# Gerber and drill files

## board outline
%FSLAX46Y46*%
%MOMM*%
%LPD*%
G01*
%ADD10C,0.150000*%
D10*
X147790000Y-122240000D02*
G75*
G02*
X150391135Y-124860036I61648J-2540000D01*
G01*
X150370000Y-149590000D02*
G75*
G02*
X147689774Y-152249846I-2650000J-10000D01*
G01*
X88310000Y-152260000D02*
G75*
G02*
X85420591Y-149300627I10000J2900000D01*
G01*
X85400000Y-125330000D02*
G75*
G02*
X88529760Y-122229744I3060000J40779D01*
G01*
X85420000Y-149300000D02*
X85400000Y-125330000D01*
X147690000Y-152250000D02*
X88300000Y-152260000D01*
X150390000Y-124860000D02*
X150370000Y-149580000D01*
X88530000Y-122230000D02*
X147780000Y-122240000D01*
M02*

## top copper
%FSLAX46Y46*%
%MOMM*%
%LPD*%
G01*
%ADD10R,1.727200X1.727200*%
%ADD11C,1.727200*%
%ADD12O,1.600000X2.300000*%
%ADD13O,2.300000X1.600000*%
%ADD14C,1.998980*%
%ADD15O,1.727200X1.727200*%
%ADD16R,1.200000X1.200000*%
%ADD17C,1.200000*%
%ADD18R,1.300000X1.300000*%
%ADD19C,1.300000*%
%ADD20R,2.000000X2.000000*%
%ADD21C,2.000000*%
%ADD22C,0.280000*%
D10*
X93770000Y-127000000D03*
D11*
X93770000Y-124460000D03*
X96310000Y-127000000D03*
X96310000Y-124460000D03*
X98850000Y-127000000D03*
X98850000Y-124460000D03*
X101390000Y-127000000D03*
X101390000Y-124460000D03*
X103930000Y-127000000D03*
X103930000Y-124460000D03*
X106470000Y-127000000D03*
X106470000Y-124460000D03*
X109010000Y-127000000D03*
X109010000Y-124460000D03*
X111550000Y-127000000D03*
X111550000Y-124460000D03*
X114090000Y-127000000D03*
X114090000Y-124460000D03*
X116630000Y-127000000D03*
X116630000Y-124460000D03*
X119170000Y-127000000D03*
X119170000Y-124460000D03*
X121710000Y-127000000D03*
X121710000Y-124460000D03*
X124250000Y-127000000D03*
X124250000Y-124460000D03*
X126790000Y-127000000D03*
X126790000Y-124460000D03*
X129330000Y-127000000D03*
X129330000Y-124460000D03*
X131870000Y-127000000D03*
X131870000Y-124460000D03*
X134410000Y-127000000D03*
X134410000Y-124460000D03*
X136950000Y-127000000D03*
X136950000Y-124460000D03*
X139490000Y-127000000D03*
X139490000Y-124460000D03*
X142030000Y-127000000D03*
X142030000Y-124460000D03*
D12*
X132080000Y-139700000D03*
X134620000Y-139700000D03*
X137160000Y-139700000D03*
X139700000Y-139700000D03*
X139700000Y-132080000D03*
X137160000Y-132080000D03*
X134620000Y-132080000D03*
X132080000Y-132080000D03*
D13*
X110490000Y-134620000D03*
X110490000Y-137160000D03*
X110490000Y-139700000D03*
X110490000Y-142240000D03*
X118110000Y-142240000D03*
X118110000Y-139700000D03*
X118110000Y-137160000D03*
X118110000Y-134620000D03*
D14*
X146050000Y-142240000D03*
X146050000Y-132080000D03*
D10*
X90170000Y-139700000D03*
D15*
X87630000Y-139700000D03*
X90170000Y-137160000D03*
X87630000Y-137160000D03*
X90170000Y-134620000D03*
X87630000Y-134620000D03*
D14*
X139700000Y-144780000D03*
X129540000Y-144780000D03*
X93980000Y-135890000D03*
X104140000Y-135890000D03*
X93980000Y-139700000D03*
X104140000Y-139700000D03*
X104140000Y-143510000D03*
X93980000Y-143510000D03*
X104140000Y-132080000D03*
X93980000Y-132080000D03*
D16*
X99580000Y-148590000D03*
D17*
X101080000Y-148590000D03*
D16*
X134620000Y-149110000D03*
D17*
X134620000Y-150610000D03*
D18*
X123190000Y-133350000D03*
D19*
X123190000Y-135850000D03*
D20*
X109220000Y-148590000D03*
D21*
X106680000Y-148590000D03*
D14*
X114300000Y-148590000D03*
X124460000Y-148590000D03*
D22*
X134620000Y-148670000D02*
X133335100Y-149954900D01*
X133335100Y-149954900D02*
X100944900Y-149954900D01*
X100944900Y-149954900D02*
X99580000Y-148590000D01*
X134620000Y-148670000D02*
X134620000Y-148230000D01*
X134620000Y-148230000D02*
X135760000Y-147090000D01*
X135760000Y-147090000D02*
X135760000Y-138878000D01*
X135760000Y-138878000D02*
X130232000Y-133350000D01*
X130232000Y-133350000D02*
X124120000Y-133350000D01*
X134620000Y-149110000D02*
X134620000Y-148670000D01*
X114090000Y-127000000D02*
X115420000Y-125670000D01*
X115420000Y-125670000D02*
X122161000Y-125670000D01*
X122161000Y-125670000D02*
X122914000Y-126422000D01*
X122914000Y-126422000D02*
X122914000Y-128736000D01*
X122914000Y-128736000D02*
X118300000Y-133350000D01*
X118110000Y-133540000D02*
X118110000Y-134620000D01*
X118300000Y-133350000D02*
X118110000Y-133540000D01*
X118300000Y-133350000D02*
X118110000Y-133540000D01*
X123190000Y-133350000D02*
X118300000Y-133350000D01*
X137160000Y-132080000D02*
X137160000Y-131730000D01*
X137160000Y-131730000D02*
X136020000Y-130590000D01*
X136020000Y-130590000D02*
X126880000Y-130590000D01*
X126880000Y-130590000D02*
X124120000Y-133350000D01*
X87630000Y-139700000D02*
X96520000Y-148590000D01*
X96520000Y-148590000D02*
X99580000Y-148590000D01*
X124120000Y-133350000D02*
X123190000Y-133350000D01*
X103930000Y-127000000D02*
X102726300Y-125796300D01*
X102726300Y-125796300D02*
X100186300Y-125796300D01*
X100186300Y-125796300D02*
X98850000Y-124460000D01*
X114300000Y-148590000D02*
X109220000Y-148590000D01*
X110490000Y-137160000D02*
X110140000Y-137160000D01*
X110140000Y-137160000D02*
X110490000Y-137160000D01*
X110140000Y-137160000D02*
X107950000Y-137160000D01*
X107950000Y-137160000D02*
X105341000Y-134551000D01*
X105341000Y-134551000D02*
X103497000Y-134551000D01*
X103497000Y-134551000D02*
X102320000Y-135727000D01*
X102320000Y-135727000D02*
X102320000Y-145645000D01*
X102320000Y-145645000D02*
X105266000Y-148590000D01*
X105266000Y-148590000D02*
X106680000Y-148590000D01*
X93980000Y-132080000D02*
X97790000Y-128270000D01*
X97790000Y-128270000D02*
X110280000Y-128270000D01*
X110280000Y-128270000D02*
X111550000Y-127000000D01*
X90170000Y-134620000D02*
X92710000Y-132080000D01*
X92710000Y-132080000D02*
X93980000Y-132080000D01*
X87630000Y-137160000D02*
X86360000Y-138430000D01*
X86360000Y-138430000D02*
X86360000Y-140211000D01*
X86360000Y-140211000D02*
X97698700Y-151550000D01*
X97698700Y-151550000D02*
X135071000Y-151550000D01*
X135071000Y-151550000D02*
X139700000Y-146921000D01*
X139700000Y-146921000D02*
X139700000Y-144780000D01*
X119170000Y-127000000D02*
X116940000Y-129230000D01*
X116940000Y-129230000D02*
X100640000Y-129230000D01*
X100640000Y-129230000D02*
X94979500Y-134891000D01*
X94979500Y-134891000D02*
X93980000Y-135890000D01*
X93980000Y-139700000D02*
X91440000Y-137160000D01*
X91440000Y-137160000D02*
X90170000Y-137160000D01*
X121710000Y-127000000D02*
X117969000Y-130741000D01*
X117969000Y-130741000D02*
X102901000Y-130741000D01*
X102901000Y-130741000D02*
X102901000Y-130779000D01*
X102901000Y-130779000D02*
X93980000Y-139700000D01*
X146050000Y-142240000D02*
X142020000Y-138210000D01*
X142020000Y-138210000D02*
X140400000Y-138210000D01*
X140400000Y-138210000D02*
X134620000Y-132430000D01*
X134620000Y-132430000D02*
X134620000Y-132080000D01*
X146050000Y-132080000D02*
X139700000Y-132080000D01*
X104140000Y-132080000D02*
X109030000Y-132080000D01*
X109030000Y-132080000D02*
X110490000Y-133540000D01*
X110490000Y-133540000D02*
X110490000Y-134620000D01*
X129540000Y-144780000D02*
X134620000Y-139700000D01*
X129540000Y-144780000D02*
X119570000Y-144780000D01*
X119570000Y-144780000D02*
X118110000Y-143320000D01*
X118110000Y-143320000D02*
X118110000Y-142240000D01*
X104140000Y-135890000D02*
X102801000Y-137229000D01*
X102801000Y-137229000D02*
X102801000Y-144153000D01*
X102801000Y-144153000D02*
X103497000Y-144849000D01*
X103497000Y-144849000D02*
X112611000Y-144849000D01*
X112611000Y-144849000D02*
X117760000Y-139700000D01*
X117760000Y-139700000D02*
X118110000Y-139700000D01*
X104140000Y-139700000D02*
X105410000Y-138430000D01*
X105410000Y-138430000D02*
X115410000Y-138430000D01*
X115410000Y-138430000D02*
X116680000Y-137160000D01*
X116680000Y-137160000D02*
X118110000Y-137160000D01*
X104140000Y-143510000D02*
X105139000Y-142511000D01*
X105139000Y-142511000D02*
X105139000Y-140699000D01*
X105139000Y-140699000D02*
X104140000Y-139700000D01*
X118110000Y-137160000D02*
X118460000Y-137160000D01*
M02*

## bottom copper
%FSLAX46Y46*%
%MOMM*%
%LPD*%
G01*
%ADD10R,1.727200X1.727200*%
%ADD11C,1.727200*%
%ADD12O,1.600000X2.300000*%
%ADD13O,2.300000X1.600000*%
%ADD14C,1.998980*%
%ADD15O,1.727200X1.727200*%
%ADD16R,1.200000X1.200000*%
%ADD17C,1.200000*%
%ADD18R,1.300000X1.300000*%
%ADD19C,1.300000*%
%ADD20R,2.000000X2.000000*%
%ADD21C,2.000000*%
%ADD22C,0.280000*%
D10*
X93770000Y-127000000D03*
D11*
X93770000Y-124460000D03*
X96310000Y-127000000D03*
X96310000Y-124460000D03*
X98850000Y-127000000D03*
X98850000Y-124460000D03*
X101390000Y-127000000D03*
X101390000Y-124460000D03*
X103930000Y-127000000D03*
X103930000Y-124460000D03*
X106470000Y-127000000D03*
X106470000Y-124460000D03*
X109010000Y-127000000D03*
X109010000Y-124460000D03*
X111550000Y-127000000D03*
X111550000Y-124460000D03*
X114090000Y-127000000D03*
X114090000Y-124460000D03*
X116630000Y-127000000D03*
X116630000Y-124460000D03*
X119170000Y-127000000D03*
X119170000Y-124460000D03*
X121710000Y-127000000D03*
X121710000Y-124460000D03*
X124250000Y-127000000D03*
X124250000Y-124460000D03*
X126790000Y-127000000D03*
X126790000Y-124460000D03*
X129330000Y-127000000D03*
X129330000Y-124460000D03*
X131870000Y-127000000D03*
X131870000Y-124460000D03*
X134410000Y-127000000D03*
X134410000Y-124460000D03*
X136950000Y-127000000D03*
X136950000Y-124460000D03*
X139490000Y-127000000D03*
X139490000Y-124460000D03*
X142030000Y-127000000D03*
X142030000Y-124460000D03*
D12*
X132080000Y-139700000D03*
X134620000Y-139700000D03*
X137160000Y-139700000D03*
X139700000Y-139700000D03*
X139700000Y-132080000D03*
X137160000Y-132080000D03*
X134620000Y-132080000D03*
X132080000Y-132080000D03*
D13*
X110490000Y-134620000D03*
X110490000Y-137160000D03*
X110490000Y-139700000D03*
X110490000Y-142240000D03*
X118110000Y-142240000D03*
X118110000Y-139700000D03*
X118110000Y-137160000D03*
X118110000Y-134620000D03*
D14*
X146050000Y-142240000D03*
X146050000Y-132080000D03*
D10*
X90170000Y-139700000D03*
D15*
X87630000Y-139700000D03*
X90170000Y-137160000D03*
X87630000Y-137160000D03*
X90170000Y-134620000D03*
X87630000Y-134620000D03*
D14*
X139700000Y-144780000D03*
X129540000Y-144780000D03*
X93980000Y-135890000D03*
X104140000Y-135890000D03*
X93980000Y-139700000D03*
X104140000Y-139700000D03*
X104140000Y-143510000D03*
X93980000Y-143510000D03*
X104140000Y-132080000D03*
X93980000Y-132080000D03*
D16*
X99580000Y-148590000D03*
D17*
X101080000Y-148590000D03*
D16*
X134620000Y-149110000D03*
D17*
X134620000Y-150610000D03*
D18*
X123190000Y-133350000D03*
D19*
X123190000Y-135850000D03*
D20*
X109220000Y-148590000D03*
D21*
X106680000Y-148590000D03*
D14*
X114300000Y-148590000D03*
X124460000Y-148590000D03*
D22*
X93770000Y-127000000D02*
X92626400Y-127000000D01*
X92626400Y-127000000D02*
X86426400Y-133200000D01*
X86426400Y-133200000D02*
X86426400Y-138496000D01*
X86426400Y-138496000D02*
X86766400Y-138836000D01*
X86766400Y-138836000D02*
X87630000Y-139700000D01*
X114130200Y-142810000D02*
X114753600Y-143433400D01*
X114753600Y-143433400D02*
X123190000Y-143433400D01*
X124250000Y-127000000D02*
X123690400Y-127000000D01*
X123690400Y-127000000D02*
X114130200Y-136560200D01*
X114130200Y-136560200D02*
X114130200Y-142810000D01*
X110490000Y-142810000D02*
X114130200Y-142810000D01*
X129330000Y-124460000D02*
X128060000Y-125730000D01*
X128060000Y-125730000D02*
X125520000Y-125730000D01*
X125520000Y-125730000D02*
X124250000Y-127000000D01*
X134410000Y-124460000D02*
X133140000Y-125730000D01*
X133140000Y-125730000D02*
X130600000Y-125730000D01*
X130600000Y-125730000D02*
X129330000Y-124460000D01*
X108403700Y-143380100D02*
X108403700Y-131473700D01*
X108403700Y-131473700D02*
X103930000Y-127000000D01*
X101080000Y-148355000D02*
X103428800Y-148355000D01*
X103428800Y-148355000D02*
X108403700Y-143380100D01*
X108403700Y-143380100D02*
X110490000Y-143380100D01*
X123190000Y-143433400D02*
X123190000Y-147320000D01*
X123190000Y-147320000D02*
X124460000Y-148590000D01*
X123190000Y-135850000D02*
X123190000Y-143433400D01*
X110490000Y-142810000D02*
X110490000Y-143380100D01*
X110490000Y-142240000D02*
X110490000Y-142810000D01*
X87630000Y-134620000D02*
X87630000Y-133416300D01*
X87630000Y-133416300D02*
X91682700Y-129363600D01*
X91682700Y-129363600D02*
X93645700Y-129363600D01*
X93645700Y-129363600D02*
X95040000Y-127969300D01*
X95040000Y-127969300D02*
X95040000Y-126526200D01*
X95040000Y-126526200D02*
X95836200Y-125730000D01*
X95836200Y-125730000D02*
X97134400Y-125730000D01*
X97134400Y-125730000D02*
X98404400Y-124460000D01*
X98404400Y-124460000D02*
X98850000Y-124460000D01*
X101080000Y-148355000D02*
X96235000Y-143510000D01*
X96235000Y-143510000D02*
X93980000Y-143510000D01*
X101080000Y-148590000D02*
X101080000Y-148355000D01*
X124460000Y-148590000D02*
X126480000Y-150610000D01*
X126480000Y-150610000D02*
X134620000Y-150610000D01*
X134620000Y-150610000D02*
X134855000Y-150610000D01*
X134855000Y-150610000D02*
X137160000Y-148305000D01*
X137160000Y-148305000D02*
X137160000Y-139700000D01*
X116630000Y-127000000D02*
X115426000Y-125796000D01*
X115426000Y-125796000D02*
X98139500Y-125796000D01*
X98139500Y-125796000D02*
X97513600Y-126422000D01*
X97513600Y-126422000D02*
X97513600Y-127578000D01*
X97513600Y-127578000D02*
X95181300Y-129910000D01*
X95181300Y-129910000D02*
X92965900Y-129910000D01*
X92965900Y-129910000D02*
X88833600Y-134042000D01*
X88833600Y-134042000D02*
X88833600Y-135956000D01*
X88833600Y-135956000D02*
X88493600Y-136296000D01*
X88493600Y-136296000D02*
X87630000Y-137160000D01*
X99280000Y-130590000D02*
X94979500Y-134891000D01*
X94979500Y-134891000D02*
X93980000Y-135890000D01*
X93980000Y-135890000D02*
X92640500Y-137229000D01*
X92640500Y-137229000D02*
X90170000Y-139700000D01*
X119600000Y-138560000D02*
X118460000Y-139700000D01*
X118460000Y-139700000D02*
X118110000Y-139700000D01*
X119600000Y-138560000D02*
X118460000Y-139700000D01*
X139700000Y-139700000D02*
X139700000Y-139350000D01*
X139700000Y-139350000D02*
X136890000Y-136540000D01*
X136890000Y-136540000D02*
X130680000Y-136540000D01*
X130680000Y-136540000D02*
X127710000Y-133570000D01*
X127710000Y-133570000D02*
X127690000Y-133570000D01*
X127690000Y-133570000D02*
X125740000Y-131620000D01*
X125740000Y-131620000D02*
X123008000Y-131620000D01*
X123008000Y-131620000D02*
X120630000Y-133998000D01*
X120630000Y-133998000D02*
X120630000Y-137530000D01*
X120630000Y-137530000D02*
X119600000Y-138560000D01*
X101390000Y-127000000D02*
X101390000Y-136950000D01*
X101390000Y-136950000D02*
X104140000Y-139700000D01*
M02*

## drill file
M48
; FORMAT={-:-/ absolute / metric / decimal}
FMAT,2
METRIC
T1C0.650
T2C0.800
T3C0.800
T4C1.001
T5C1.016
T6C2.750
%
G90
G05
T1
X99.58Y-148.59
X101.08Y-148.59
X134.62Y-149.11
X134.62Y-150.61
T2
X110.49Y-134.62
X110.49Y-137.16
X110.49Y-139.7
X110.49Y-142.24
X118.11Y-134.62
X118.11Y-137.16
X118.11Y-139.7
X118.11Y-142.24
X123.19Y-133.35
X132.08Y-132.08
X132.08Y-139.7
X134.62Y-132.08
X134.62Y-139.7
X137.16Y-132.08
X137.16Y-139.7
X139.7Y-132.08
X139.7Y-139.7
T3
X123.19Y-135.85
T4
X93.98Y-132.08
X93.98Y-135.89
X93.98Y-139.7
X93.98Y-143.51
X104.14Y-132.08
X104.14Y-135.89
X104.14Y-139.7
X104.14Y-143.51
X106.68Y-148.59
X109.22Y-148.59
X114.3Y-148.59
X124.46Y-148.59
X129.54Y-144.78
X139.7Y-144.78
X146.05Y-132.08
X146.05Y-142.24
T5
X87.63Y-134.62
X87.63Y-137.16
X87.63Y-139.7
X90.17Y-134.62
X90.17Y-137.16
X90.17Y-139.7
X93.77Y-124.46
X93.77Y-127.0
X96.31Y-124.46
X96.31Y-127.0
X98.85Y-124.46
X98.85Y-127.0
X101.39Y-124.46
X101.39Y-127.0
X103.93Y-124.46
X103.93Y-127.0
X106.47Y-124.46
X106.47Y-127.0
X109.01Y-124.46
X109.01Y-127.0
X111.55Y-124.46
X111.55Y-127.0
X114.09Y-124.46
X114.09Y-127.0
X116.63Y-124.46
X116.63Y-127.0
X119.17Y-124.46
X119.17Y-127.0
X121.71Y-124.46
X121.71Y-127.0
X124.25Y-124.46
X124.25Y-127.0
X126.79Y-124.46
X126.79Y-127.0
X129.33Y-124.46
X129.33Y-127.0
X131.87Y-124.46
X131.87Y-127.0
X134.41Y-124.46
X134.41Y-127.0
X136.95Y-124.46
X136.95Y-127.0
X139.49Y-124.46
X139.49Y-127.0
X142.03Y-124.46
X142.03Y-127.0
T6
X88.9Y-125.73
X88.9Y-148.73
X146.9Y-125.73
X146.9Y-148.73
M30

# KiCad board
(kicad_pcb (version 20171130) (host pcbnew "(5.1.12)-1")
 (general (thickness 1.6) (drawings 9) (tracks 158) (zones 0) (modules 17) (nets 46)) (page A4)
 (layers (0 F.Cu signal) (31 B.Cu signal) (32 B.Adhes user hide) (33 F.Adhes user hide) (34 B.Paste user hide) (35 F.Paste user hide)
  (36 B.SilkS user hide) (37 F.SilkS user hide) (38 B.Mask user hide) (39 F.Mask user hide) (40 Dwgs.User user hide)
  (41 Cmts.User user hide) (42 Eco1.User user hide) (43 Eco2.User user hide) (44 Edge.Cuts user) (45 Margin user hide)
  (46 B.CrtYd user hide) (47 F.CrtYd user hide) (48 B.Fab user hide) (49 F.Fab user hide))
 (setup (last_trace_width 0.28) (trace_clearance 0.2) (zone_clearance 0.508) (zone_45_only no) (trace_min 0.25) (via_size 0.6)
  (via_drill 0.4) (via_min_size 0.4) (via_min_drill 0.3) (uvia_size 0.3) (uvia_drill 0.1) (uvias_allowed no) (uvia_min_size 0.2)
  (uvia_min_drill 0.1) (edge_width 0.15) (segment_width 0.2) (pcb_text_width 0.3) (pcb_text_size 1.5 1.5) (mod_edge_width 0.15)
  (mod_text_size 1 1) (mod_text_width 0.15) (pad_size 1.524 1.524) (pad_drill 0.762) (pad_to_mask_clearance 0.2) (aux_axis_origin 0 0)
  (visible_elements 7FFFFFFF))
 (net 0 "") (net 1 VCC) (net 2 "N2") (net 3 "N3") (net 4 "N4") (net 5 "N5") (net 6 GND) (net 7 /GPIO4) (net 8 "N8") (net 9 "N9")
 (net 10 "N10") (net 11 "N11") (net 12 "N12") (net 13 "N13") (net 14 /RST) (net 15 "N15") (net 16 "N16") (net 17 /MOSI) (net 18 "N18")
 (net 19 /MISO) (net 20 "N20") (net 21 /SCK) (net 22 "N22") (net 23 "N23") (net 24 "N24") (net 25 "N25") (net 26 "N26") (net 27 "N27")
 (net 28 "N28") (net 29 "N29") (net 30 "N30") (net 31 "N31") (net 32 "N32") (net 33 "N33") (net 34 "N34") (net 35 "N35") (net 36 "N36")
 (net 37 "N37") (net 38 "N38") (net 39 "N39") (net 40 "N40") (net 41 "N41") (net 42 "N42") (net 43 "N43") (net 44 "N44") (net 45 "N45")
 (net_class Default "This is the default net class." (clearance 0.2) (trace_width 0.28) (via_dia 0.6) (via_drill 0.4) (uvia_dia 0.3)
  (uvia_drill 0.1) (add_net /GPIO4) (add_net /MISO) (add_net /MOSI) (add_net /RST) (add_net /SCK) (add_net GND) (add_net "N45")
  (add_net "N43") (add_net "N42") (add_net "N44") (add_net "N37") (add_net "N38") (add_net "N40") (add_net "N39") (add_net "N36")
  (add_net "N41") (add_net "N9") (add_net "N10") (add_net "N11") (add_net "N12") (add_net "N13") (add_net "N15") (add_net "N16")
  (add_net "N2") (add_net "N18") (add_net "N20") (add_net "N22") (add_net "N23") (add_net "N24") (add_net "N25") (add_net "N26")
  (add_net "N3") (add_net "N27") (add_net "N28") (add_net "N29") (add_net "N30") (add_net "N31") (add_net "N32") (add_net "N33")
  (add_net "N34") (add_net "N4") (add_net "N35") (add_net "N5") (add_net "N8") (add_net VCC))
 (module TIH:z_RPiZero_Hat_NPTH (layer F.Cu) (at 117.9 137.23)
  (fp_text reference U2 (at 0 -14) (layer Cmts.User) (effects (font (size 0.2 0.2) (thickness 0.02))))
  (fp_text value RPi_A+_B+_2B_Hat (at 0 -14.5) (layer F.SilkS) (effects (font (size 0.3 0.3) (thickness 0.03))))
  (pad "" smd circle (at 29 -11.5) (size 6 6) (layers *.Mask)) (pad "" smd circle (at 29 11.5) (size 6 6) (layers *.Mask))
  (pad "" smd circle (at -29 -11.5) (size 6 6) (layers *.Mask))
  (pad "" np_thru_hole circle (at -29 11.5) (size 2.75 2.75) (drill 2.75) (layers *.Cu *.Mask) (solder_paste_margin 0.001))
  (pad "" np_thru_hole circle (at 29 -11.5) (size 2.75 2.75) (drill 2.75) (layers *.Cu *.Mask) (solder_paste_margin 0.001))
  (pad "" np_thru_hole circle (at -29 -11.5) (size 2.75 2.75) (drill 2.75) (layers *.Cu *.Mask) (solder_paste_margin 0.001))
  (pad "" np_thru_hole circle (at 29 11.5) (size 2.75 2.75) (drill 2.75) (layers *.Cu *.Mask) (solder_paste_margin 0.001))
  (pad 1 thru_hole rect (at -24.13 -10.23 180) (size 1.7272 1.7272) (drill 1.016) (layers *.Cu *.Mask F.SilkS) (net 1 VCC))
  (pad 2 thru_hole circle (at -24.13 -12.77 180) (size 1.7272 1.7272) (drill 1.016) (layers *.Cu *.Mask F.SilkS) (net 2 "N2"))
  (pad 3 thru_hole circle (at -21.59 -10.23 180) (size 1.7272 1.7272) (drill 1.016) (layers *.Cu *.Mask F.SilkS) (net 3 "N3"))
  (pad 4 thru_hole circle (at -21.59 -12.77 180) (size 1.7272 1.7272) (drill 1.016) (layers *.Cu *.Mask F.SilkS) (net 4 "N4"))
  (pad 5 thru_hole circle (at -19.05 -10.23 180) (size 1.7272 1.7272) (drill 1.016) (layers *.Cu *.Mask F.SilkS) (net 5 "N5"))
  (pad 6 thru_hole circle (at -19.05 -12.77 180) (size 1.7272 1.7272) (drill 1.016) (layers *.Cu *.Mask F.SilkS) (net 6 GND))
  (pad 7 thru_hole circle (at -16.51 -10.23 180) (size 1.7272 1.7272) (drill 1.016) (layers *.Cu *.Mask F.SilkS) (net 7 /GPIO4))
  (pad 8 thru_hole circle (at -16.51 -12.77 180) (size 1.7272 1.7272) (drill 1.016) (layers *.Cu *.Mask F.SilkS) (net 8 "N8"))
  (pad 9 thru_hole circle (at -13.97 -10.23 180) (size 1.7272 1.7272) (drill 1.016) (layers *.Cu *.Mask F.SilkS) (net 6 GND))
  (pad 10 thru_hole circle (at -13.97 -12.77 180) (size 1.7272 1.7272) (drill 1.016) (layers *.Cu *.Mask F.SilkS) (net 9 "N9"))
  (pad 11 thru_hole circle (at -11.43 -10.23 180) (size 1.7272 1.7272) (drill 1.016) (layers *.Cu *.Mask F.SilkS) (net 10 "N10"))
  (pad 12 thru_hole circle (at -11.43 -12.77 180) (size 1.7272 1.7272) (drill 1.016) (layers *.Cu *.Mask F.SilkS) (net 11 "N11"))
  (pad 13 thru_hole circle (at -8.89 -10.23 180) (size 1.7272 1.7272) (drill 1.016) (layers *.Cu *.Mask F.SilkS) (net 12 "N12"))
  (pad 14 thru_hole circle (at -8.89 -12.77 180) (size 1.7272 1.7272) (drill 1.016) (layers *.Cu *.Mask F.SilkS) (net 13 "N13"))
  (pad 15 thru_hole circle (at -6.35 -10.23 180) (size 1.7272 1.7272) (drill 1.016) (layers *.Cu *.Mask F.SilkS) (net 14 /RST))
  (pad 16 thru_hole circle (at -6.35 -12.77 180) (size 1.7272 1.7272) (drill 1.016) (layers *.Cu *.Mask F.SilkS) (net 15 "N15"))
  (pad 17 thru_hole circle (at -3.81 -10.23 180) (size 1.7272 1.7272) (drill 1.016) (layers *.Cu *.Mask F.SilkS) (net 1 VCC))
  (pad 18 thru_hole circle (at -3.81 -12.77 180) (size 1.7272 1.7272) (drill 1.016) (layers *.Cu *.Mask F.SilkS) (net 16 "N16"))
  (pad 19 thru_hole circle (at -1.27 -10.23 180) (size 1.7272 1.7272) (drill 1.016) (layers *.Cu *.Mask F.SilkS) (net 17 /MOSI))
  (pad 20 thru_hole circle (at -1.27 -12.77 180) (size 1.7272 1.7272) (drill 1.016) (layers *.Cu *.Mask F.SilkS) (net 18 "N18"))
  (pad 21 thru_hole circle (at 1.27 -10.23 180) (size 1.7272 1.7272) (drill 1.016) (layers *.Cu *.Mask F.SilkS) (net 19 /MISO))
  (pad 22 thru_hole circle (at 1.27 -12.77 180) (size 1.7272 1.7272) (drill 1.016) (layers *.Cu *.Mask F.SilkS) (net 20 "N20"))
  (pad 23 thru_hole circle (at 3.81 -10.23 180) (size 1.7272 1.7272) (drill 1.016) (layers *.Cu *.Mask F.SilkS) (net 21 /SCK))
  (pad 24 thru_hole circle (at 3.81 -12.77 180) (size 1.7272 1.7272) (drill 1.016) (layers *.Cu *.Mask F.SilkS) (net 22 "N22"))
  (pad 25 thru_hole circle (at 6.35 -10.23 180) (size 1.7272 1.7272) (drill 1.016) (layers *.Cu *.Mask F.SilkS) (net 6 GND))
  (pad 26 thru_hole circle (at 6.35 -12.77 180) (size 1.7272 1.7272) (drill 1.016) (layers *.Cu *.Mask F.SilkS) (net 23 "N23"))
  (pad 27 thru_hole circle (at 8.89 -10.23 180) (size 1.7272 1.7272) (drill 1.016) (layers *.Cu *.Mask F.SilkS) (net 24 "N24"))
  (pad 28 thru_hole circle (at 8.89 -12.77 180) (size 1.7272 1.7272) (drill 1.016) (layers *.Cu *.Mask F.SilkS) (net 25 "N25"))
  (pad 29 thru_hole circle (at 11.43 -10.23 180) (size 1.7272 1.7272) (drill 1.016) (layers *.Cu *.Mask F.SilkS) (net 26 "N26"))
  (pad 30 thru_hole circle (at 11.43 -12.77 180) (size 1.7272 1.7272) (drill 1.016) (layers *.Cu *.Mask F.SilkS) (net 6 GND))
  (pad 31 thru_hole circle (at 13.97 -10.23 180) (size 1.7272 1.7272) (drill 1.016) (layers *.Cu *.Mask F.SilkS) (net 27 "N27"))
  (pad 32 thru_hole circle (at 13.97 -12.77 180) (size 1.7272 1.7272) (drill 1.016) (layers *.Cu *.Mask F.SilkS) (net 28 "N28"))
  (pad 33 thru_hole circle (at 16.51 -10.23 180) (size 1.7272 1.7272) (drill 1.016) (layers *.Cu *.Mask F.SilkS) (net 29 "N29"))
  (pad 34 thru_hole circle (at 16.51 -12.77 180) (size 1.7272 1.7272) (drill 1.016) (layers *.Cu *.Mask F.SilkS) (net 6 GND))
  (pad 35 thru_hole circle (at 19.05 -10.23 180) (size 1.7272 1.7272) (drill 1.016) (layers *.Cu *.Mask F.SilkS) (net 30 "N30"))
  (pad 36 thru_hole circle (at 19.05 -12.77 180) (size 1.7272 1.7272) (drill 1.016) (layers *.Cu *.Mask F.SilkS) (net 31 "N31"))
  (pad 37 thru_hole circle (at 21.59 -10.23 180) (size 1.7272 1.7272) (drill 1.016) (layers *.Cu *.Mask F.SilkS) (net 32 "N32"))
  (pad 38 thru_hole circle (at 21.59 -12.77 180) (size 1.7272 1.7272) (drill 1.016) (layers *.Cu *.Mask F.SilkS) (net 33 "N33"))
  (pad 39 thru_hole circle (at 24.13 -10.23 180) (size 1.7272 1.7272) (drill 1.016) (layers *.Cu *.Mask F.SilkS) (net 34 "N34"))
  (pad 40 thru_hole circle (at 24.13 -12.77 180) (size 1.7272 1.7272) (drill 1.016) (layers *.Cu *.Mask F.SilkS) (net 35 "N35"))
  (pad "" smd circle (at -29 11.5) (size 6 6) (layers *.Mask)))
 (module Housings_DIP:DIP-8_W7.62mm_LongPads (layer F.Cu) (at 132.08 139.7 90)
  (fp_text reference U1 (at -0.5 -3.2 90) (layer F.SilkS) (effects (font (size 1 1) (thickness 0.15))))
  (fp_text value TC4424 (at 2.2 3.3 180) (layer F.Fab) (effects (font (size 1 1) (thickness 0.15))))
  (pad 1 thru_hole oval (at 0 0 90) (size 2.3 1.6) (drill 0.8) (layers *.Cu *.Mask F.SilkS) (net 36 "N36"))
  (pad 2 thru_hole oval (at 0 2.54 90) (size 2.3 1.6) (drill 0.8) (layers *.Cu *.Mask F.SilkS) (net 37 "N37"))
  (pad 3 thru_hole oval (at 0 5.08 90) (size 2.3 1.6) (drill 0.8) (layers *.Cu *.Mask F.SilkS) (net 6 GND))
  (pad 4 thru_hole oval (at 0 7.62 90) (size 2.3 1.6) (drill 0.8) (layers *.Cu *.Mask F.SilkS) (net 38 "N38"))
  (pad 5 thru_hole oval (at 7.62 7.62 90) (size 2.3 1.6) (drill 0.8) (layers *.Cu *.Mask F.SilkS) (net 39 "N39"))
  (pad 6 thru_hole oval (at 7.62 5.08 90) (size 2.3 1.6) (drill 0.8) (layers *.Cu *.Mask F.SilkS) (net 1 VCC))
  (pad 7 thru_hole oval (at 7.62 2.54 90) (size 2.3 1.6) (drill 0.8) (layers *.Cu *.Mask F.SilkS) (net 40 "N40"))
  (pad 8 thru_hole oval (at 7.62 0 90) (size 2.3 1.6) (drill 0.8) (layers *.Cu *.Mask F.SilkS) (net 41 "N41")))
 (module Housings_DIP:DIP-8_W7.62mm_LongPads (layer F.Cu) (at 110.49 134.62)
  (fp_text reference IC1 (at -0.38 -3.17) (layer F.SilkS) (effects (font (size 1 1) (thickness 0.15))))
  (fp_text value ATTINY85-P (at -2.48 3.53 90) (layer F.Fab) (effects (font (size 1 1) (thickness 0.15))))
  (pad 1 thru_hole oval (at 0 0) (size 2.3 1.6) (drill 0.8) (layers *.Cu *.Mask F.SilkS) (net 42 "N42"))
  (pad 2 thru_hole oval (at 0 2.54) (size 2.3 1.6) (drill 0.8) (layers *.Cu *.Mask F.SilkS) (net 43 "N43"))
  (pad 3 thru_hole oval (at 0 5.08) (size 2.3 1.6) (drill 0.8) (layers *.Cu *.Mask F.SilkS) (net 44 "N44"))
  (pad 4 thru_hole oval (at 0 7.62) (size 2.3 1.6) (drill 0.8) (layers *.Cu *.Mask F.SilkS) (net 6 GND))
  (pad 5 thru_hole oval (at 7.62 7.62) (size 2.3 1.6) (drill 0.8) (layers *.Cu *.Mask F.SilkS) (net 37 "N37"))
  (pad 6 thru_hole oval (at 7.62 5.08) (size 2.3 1.6) (drill 0.8) (layers *.Cu *.Mask F.SilkS) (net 38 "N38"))
  (pad 7 thru_hole oval (at 7.62 2.54) (size 2.3 1.6) (drill 0.8) (layers *.Cu *.Mask F.SilkS) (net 7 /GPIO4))
  (pad 8 thru_hole oval (at 7.62 0) (size 2.3 1.6) (drill 0.8) (layers *.Cu *.Mask F.SilkS) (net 1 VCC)))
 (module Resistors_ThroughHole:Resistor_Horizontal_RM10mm (layer F.Cu) (at 146.05 137.16 90)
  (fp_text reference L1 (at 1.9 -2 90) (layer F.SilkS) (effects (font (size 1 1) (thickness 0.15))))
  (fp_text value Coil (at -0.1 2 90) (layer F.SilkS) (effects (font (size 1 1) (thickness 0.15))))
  (pad 1 thru_hole circle (at -5.08 0 90) (size 1.99898 1.99898) (drill 1.00076) (layers *.Cu *.SilkS *.Mask) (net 40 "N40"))
  (pad 2 thru_hole circle (at 5.08 0 90) (size 1.99898 1.99898) (drill 1.00076) (layers *.Cu *.SilkS *.Mask) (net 39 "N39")))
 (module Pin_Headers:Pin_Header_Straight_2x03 (layer F.Cu) (at 90.17 139.7 180)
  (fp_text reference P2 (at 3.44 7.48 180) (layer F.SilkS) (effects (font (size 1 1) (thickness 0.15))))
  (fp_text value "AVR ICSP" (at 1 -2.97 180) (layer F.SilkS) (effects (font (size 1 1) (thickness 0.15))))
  (pad 1 thru_hole rect (at 0 0 180) (size 1.7272 1.7272) (drill 1.016) (layers *.Cu *.Mask F.SilkS) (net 19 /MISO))
  (pad 2 thru_hole oval (at 2.54 0 180) (size 1.7272 1.7272) (drill 1.016) (layers *.Cu *.Mask F.SilkS) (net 1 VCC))
  (pad 3 thru_hole oval (at 0 2.54 180) (size 1.7272 1.7272) (drill 1.016) (layers *.Cu *.Mask F.SilkS) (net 21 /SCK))
  (pad 4 thru_hole oval (at 2.54 2.54 180) (size 1.7272 1.7272) (drill 1.016) (layers *.Cu *.Mask F.SilkS) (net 17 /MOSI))
  (pad 5 thru_hole oval (at 0 5.08 180) (size 1.7272 1.7272) (drill 1.016) (layers *.Cu *.Mask F.SilkS) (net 14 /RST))
  (pad 6 thru_hole oval (at 2.54 5.08 180) (size 1.7272 1.7272) (drill 1.016) (layers *.Cu *.Mask F.SilkS) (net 6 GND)))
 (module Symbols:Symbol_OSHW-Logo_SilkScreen (layer B.Cu) (at 99.06 135.89 180)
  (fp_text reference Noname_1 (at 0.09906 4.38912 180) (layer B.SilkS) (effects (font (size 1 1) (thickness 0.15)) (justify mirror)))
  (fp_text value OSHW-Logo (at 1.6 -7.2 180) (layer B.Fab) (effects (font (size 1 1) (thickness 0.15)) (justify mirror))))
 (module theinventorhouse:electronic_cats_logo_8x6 (layer B.Cu) (at 123.19 142.24 180)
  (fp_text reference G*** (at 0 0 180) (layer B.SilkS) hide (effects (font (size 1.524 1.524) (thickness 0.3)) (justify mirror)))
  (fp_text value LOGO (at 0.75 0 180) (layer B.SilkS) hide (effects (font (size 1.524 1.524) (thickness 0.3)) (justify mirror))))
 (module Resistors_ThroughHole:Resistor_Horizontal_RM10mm (layer F.Cu) (at 139.7 144.78 180)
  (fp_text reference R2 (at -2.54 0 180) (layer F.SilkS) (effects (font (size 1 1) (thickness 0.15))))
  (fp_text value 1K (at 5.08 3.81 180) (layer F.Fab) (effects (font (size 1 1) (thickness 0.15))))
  (pad 1 thru_hole circle (at 0 0 180) (size 1.99898 1.99898) (drill 1.00076) (layers *.Cu *.SilkS *.Mask) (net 17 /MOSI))
  (pad 2 thru_hole circle (at 10.16 0 180) (size 1.99898 1.99898) (drill 1.00076) (layers *.Cu *.SilkS *.Mask) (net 37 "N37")))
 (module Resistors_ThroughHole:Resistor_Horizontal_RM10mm (layer F.Cu) (at 93.98 135.89)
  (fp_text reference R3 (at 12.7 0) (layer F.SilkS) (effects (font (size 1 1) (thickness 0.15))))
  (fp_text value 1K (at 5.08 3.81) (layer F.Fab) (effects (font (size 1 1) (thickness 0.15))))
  (pad 1 thru_hole circle (at 0 0) (size 1.99898 1.99898) (drill 1.00076) (layers *.Cu *.SilkS *.Mask) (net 19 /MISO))
  (pad 2 thru_hole circle (at 10.16 0) (size 1.99898 1.99898) (drill 1.00076) (layers *.Cu *.SilkS *.Mask) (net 38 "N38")))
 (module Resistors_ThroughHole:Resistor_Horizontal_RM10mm (layer F.Cu) (at 93.98 139.7)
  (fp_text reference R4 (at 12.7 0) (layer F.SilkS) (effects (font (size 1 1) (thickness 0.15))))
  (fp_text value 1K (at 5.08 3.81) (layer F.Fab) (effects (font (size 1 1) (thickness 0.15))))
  (pad 1 thru_hole circle (at 0 0) (size 1.99898 1.99898) (drill 1.00076) (layers *.Cu *.SilkS *.Mask) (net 21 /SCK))
  (pad 2 thru_hole circle (at 10.16 0) (size 1.99898 1.99898) (drill 1.00076) (layers *.Cu *.SilkS *.Mask) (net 7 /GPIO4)))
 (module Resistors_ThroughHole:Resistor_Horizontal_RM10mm (layer F.Cu) (at 104.14 143.51 180)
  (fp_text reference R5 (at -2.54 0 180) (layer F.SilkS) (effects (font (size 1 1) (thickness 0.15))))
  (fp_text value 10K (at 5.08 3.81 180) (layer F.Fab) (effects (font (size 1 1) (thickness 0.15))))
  (pad 1 thru_hole circle (at 0 0 180) (size 1.99898 1.99898) (drill 1.00076) (layers *.Cu *.SilkS *.Mask) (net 7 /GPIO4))
  (pad 2 thru_hole circle (at 10.16 0 180) (size 1.99898 1.99898) (drill 1.00076) (layers *.Cu *.SilkS *.Mask) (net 6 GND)))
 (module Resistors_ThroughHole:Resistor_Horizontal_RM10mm (layer F.Cu) (at 104.14 132.08 180)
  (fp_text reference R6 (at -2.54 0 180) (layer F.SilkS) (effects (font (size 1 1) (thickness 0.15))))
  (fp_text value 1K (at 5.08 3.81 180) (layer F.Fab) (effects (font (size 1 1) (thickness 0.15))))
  (pad 1 thru_hole circle (at 0 0 180) (size 1.99898 1.99898) (drill 1.00076) (layers *.Cu *.SilkS *.Mask) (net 42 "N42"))
  (pad 2 thru_hole circle (at 10.16 0 180) (size 1.99898 1.99898) (drill 1.00076) (layers *.Cu *.SilkS *.Mask) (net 14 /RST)))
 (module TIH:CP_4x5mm (layer F.Cu) (at 100.33 148.59 270)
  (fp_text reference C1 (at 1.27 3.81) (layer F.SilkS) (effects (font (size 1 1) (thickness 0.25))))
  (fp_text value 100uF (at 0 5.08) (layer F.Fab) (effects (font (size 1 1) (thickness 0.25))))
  (pad 1 thru_hole rect (at 0 0.75 270) (size 1.2 1.2) (drill 0.65) (layers *.Cu *.Mask F.SilkS) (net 1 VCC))
  (pad 2 thru_hole circle (at 0 -0.75 270) (size 1.2 1.2) (drill 0.65) (layers *.Cu *.Mask F.SilkS) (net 6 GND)))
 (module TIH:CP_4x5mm (layer F.Cu) (at 134.62 149.86 180)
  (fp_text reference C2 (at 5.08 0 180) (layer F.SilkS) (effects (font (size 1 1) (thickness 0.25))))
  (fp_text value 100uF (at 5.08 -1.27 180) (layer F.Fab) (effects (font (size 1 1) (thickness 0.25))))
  (pad 1 thru_hole rect (at 0 0.75 180) (size 1.2 1.2) (drill 0.65) (layers *.Cu *.Mask F.SilkS) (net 1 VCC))
  (pad 2 thru_hole circle (at 0 -0.75 180) (size 1.2 1.2) (drill 0.65) (layers *.Cu *.Mask F.SilkS) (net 6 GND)))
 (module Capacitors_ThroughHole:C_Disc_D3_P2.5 (layer F.Cu) (at 123.19 133.35 270)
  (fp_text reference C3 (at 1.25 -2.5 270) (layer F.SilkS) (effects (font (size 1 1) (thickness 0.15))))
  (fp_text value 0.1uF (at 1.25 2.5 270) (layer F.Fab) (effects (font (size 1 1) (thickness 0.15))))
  (pad 1 thru_hole rect (at 0 0 270) (size 1.3 1.3) (drill 0.8) (layers *.Cu *.Mask F.SilkS) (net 1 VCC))
  (pad 2 thru_hole circle (at 2.5 0 270) (size 1.3 1.3) (drill 0.8001) (layers *.Cu *.Mask F.SilkS) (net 6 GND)))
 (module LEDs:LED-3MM (layer F.Cu) (at 109.22 148.59 180)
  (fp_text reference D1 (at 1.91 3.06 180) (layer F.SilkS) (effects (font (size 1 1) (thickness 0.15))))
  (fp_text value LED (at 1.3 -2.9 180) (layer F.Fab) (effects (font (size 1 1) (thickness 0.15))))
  (pad 1 thru_hole rect (at 0 0 270) (size 2 2) (drill 1.00076) (layers *.Cu *.Mask F.SilkS) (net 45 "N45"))
  (pad 2 thru_hole circle (at 2.54 0 180) (size 2 2) (drill 1.00076) (layers *.Cu *.Mask F.SilkS) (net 43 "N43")))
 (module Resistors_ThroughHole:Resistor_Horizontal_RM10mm (layer F.Cu) (at 114.3 148.59)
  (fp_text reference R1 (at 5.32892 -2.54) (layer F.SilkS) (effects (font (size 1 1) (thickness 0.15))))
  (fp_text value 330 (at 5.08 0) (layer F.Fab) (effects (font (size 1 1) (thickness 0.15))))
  (pad 1 thru_hole circle (at 0 0) (size 1.99898 1.99898) (drill 1.00076) (layers *.Cu *.SilkS *.Mask) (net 45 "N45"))
  (pad 2 thru_hole circle (at 10.16 0) (size 1.99898 1.99898) (drill 1.00076) (layers *.Cu *.SilkS *.Mask) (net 6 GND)))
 (gr_arc (start 147.851648 124.78) (end 147.79 122.24) (angle 93.19551596) (layer Edge.Cuts) (width 0.15))
 (gr_arc (start 147.72 149.6) (end 150.37 149.59) (angle 90.86973717) (layer Edge.Cuts) (width 0.15))
 (gr_arc (start 88.32 149.36) (end 88.31 152.26) (angle 90.97554646) (layer Edge.Cuts) (width 0.15))
 (gr_arc (start 88.46 125.289221) (end 85.4 125.33) (angle 92.06969626) (layer Edge.Cuts) (width 0.15))
 (gr_line (start 85.42 149.3) (end 85.4 125.33) (layer Edge.Cuts) (width 0.15))
 (gr_line (start 147.69 152.25) (end 88.3 152.26) (layer Edge.Cuts) (width 0.15))
 (gr_line (start 150.39 124.86) (end 150.37 149.58) (layer Edge.Cuts) (width 0.15))
 (gr_line (start 88.53 122.23) (end 147.78 122.24) (layer Edge.Cuts) (width 0.15))
 (segment (start 134.62 148.67) (end 133.3351 149.9549) (width 0.28) (layer F.Cu) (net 1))
 (segment (start 133.3351 149.9549) (end 100.9449 149.9549) (width 0.28) (layer F.Cu) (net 1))
 (segment (start 100.9449 149.9549) (end 99.58 148.59) (width 0.28) (layer F.Cu) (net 1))
 (segment (start 134.62 148.67) (end 134.62 148.23) (width 0.28) (layer F.Cu) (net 1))
 (segment (start 134.62 148.23) (end 135.76 147.09) (width 0.28) (layer F.Cu) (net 1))
 (segment (start 135.76 147.09) (end 135.76 138.878) (width 0.28) (layer F.Cu) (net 1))
 (segment (start 135.76 138.878) (end 130.232 133.35) (width 0.28) (layer F.Cu) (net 1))
 (segment (start 130.232 133.35) (end 124.12 133.35) (width 0.28) (layer F.Cu) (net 1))
 (segment (start 134.62 149.11) (end 134.62 148.67) (width 0.28) (layer F.Cu) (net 1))
 (segment (start 114.09 127) (end 115.42 125.67) (width 0.28) (layer F.Cu) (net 1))
 (segment (start 115.42 125.67) (end 122.161 125.67) (width 0.28) (layer F.Cu) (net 1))
 (segment (start 122.161 125.67) (end 122.914 126.422) (width 0.28) (layer F.Cu) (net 1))
 (segment (start 122.914 126.422) (end 122.914 128.736) (width 0.28) (layer F.Cu) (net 1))
 (segment (start 122.914 128.736) (end 118.3 133.35) (width 0.28) (layer F.Cu) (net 1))
 (segment (start 118.11 133.54) (end 118.11 134.62) (width 0.28) (layer F.Cu) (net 1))
 (segment (start 118.3 133.35) (end 118.11 133.54) (width 0.28) (layer F.Cu) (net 1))
 (segment (start 118.3 133.35) (end 118.11 133.54) (width 0.28) (layer F.Cu) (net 1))
 (segment (start 123.19 133.35) (end 118.3 133.35) (width 0.28) (layer F.Cu) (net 1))
 (segment (start 137.16 132.08) (end 137.16 131.73) (width 0.28) (layer F.Cu) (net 1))
 (segment (start 137.16 131.73) (end 136.02 130.59) (width 0.28) (layer F.Cu) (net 1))
 (segment (start 136.02 130.59) (end 126.88 130.59) (width 0.28) (layer F.Cu) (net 1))
 (segment (start 126.88 130.59) (end 124.12 133.35) (width 0.28) (layer F.Cu) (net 1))
 (segment (start 87.63 139.7) (end 96.52 148.59) (width 0.28) (layer F.Cu) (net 1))
 (segment (start 96.52 148.59) (end 99.58 148.59) (width 0.28) (layer F.Cu) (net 1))
 (segment (start 124.12 133.35) (end 123.19 133.35) (width 0.28) (layer F.Cu) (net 1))
 (segment (start 93.77 127) (end 92.6264 127) (width 0.28) (layer B.Cu) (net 1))
 (segment (start 92.6264 127) (end 86.4264 133.2) (width 0.28) (layer B.Cu) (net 1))
 (segment (start 86.4264 133.2) (end 86.4264 138.496) (width 0.28) (layer B.Cu) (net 1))
 (segment (start 86.4264 138.496) (end 86.7664 138.836) (width 0.28) (layer B.Cu) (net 1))
 (segment (start 86.7664 138.836) (end 87.63 139.7) (width 0.28) (layer B.Cu) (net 1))
 (segment (start 103.93 127) (end 102.7263 125.7963) (width 0.28) (layer F.Cu) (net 6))
 (segment (start 102.7263 125.7963) (end 100.1863 125.7963) (width 0.28) (layer F.Cu) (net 6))
 (segment (start 100.1863 125.7963) (end 98.85 124.46) (width 0.28) (layer F.Cu) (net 6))
 (segment (start 114.1302 142.81) (end 114.7536 143.4334) (width 0.28) (layer B.Cu) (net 6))
 (segment (start 114.7536 143.4334) (end 123.19 143.4334) (width 0.28) (layer B.Cu) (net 6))
 (segment (start 124.25 127) (end 123.6904 127) (width 0.28) (layer B.Cu) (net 6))
 (segment (start 123.6904 127) (end 114.1302 136.5602) (width 0.28) (layer B.Cu) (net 6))
 (segment (start 114.1302 136.5602) (end 114.1302 142.81) (width 0.28) (layer B.Cu) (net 6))
 (segment (start 110.49 142.81) (end 114.1302 142.81) (width 0.28) (layer B.Cu) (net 6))
 (segment (start 129.33 124.46) (end 128.06 125.73) (width 0.28) (layer B.Cu) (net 6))
 (segment (start 128.06 125.73) (end 125.52 125.73) (width 0.28) (layer B.Cu) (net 6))
 (segment (start 125.52 125.73) (end 124.25 127) (width 0.28) (layer B.Cu) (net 6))
 (segment (start 134.41 124.46) (end 133.14 125.73) (width 0.28) (layer B.Cu) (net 6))
 (segment (start 133.14 125.73) (end 130.6 125.73) (width 0.28) (layer B.Cu) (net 6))
 (segment (start 130.6 125.73) (end 129.33 124.46) (width 0.28) (layer B.Cu) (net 6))
 (segment (start 108.4037 143.3801) (end 108.4037 131.4737) (width 0.28) (layer B.Cu) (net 6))
 (segment (start 108.4037 131.4737) (end 103.93 127) (width 0.28) (layer B.Cu) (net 6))
 (segment (start 101.08 148.355) (end 103.4288 148.355) (width 0.28) (layer B.Cu) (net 6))
 (segment (start 103.4288 148.355) (end 108.4037 143.3801) (width 0.28) (layer B.Cu) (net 6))
 (segment (start 108.4037 143.3801) (end 110.49 143.3801) (width 0.28) (layer B.Cu) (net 6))
 (segment (start 123.19 143.4334) (end 123.19 147.32) (width 0.28) (layer B.Cu) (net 6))
 (segment (start 123.19 147.32) (end 124.46 148.59) (width 0.28) (layer B.Cu) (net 6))
 (segment (start 123.19 135.85) (end 123.19 143.4334) (width 0.28) (layer B.Cu) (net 6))
 (segment (start 110.49 142.81) (end 110.49 143.3801) (width 0.28) (layer B.Cu) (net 6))
 (segment (start 110.49 142.24) (end 110.49 142.81) (width 0.28) (layer B.Cu) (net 6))
 (segment (start 87.63 134.62) (end 87.63 133.4163) (width 0.28) (layer B.Cu) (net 6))
 (segment (start 87.63 133.4163) (end 91.6827 129.3636) (width 0.28) (layer B.Cu) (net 6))
 (segment (start 91.6827 129.3636) (end 93.6457 129.3636) (width 0.28) (layer B.Cu) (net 6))
 (segment (start 93.6457 129.3636) (end 95.04 127.9693) (width 0.28) (layer B.Cu) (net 6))
 (segment (start 95.04 127.9693) (end 95.04 126.5262) (width 0.28) (layer B.Cu) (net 6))
 (segment (start 95.04 126.5262) (end 95.8362 125.73) (width 0.28) (layer B.Cu) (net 6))
 (segment (start 95.8362 125.73) (end 97.1344 125.73) (width 0.28) (layer B.Cu) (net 6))
 (segment (start 97.1344 125.73) (end 98.4044 124.46) (width 0.28) (layer B.Cu) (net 6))
 (segment (start 98.4044 124.46) (end 98.85 124.46) (width 0.28) (layer B.Cu) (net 6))
 (segment (start 101.08 148.355) (end 96.235 143.51) (width 0.28) (layer B.Cu) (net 6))
 (segment (start 96.235 143.51) (end 93.98 143.51) (width 0.28) (layer B.Cu) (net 6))
 (segment (start 101.08 148.59) (end 101.08 148.355) (width 0.28) (layer B.Cu) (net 6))
 (segment (start 124.46 148.59) (end 126.48 150.61) (width 0.28) (layer B.Cu) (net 6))
 (segment (start 126.48 150.61) (end 134.62 150.61) (width 0.28) (layer B.Cu) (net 6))
 (segment (start 134.62 150.61) (end 134.855 150.61) (width 0.28) (layer B.Cu) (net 6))
 (segment (start 134.855 150.61) (end 137.16 148.305) (width 0.28) (layer B.Cu) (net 6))
 (segment (start 137.16 148.305) (end 137.16 139.7) (width 0.28) (layer B.Cu) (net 6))
 (segment (start 114.3 148.59) (end 109.22 148.59) (width 0.28) (layer F.Cu) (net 45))
 (segment (start 110.49 137.16) (end 110.14 137.16) (width 0.28) (layer F.Cu) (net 43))
 (segment (start 110.14 137.16) (end 110.49 137.16) (width 0.28) (layer F.Cu) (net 43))
 (segment (start 110.14 137.16) (end 107.95 137.16) (width 0.28) (layer F.Cu) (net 43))
 (segment (start 107.95 137.16) (end 105.341 134.551) (width 0.28) (layer F.Cu) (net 43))
 (segment (start 105.341 134.551) (end 103.497 134.551) (width 0.28) (layer F.Cu) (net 43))
 (segment (start 103.497 134.551) (end 102.32 135.727) (width 0.28) (layer F.Cu) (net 43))
 (segment (start 102.32 135.727) (end 102.32 145.645) (width 0.28) (layer F.Cu) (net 43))
 (segment (start 102.32 145.645) (end 105.266 148.59) (width 0.28) (layer F.Cu) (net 43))
 (segment (start 105.266 148.59) (end 106.68 148.59) (width 0.28) (layer F.Cu) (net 43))
 (segment (start 93.98 132.08) (end 97.79 128.27) (width 0.28) (layer F.Cu) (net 14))
 (segment (start 97.79 128.27) (end 110.28 128.27) (width 0.28) (layer F.Cu) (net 14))
 (segment (start 110.28 128.27) (end 111.55 127) (width 0.28) (layer F.Cu) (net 14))
 (segment (start 90.17 134.62) (end 92.71 132.08) (width 0.28) (layer F.Cu) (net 14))
 (segment (start 92.71 132.08) (end 93.98 132.08) (width 0.28) (layer F.Cu) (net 14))
 (segment (start 87.63 137.16) (end 86.36 138.43) (width 0.28) (layer F.Cu) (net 17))
 (segment (start 86.36 138.43) (end 86.36 140.211) (width 0.28) (layer F.Cu) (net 17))
 (segment (start 86.36 140.211) (end 97.6987 151.55) (width 0.28) (layer F.Cu) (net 17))
 (segment (start 97.6987 151.55) (end 135.071 151.55) (width 0.28) (layer F.Cu) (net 17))
 (segment (start 135.071 151.55) (end 139.7 146.921) (width 0.28) (layer F.Cu) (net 17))
 (segment (start 139.7 146.921) (end 139.7 144.78) (width 0.28) (layer F.Cu) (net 17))
 (segment (start 116.63 127) (end 115.426 125.796) (width 0.28) (layer B.Cu) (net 17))
 (segment (start 115.426 125.796) (end 98.1395 125.796) (width 0.28) (layer B.Cu) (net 17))
 (segment (start 98.1395 125.796) (end 97.5136 126.422) (width 0.28) (layer B.Cu) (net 17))
 (segment (start 97.5136 126.422) (end 97.5136 127.578) (width 0.28) (layer B.Cu) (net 17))
 (segment (start 97.5136 127.578) (end 95.1813 129.91) (width 0.28) (layer B.Cu) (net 17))
 (segment (start 95.1813 129.91) (end 92.9659 129.91) (width 0.28) (layer B.Cu) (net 17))
 (segment (start 92.9659 129.91) (end 88.8336 134.042) (width 0.28) (layer B.Cu) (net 17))
 (segment (start 88.8336 134.042) (end 88.8336 135.956) (width 0.28) (layer B.Cu) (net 17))
 (segment (start 88.8336 135.956) (end 88.4936 136.296) (width 0.28) (layer B.Cu) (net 17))
 (segment (start 88.4936 136.296) (end 87.63 137.16) (width 0.28) (layer B.Cu) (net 17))
 (segment (start 99.28 130.59) (end 94.9795 134.891) (width 0.28) (layer B.Cu) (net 19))
 (segment (start 94.9795 134.891) (end 93.98 135.89) (width 0.28) (layer B.Cu) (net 19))
 (segment (start 93.98 135.89) (end 92.6405 137.229) (width 0.28) (layer B.Cu) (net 19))
 (segment (start 92.6405 137.229) (end 90.17 139.7) (width 0.28) (layer B.Cu) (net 19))
 (segment (start 119.17 127) (end 116.94 129.23) (width 0.28) (layer F.Cu) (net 19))
 (segment (start 116.94 129.23) (end 100.64 129.23) (width 0.28) (layer F.Cu) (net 19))
 (segment (start 100.64 129.23) (end 94.9795 134.891) (width 0.28) (layer F.Cu) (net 19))
 (segment (start 94.9795 134.891) (end 93.98 135.89) (width 0.28) (layer F.Cu) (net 19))
 (segment (start 93.98 139.7) (end 91.44 137.16) (width 0.28) (layer F.Cu) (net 21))
 (segment (start 91.44 137.16) (end 90.17 137.16) (width 0.28) (layer F.Cu) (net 21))
 (segment (start 121.71 127) (end 117.969 130.741) (width 0.28) (layer F.Cu) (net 21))
 (segment (start 117.969 130.741) (end 102.901 130.741) (width 0.28) (layer F.Cu) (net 21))
 (segment (start 102.901 130.741) (end 102.901 130.779) (width 0.28) (layer F.Cu) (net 21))
 (segment (start 102.901 130.779) (end 93.98 139.7) (width 0.28) (layer F.Cu) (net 21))
 (segment (start 146.05 142.24) (end 142.02 138.21) (width 0.28) (layer F.Cu) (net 40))
 (segment (start 142.02 138.21) (end 140.4 138.21) (width 0.28) (layer F.Cu) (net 40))
 (segment (start 140.4 138.21) (end 134.62 132.43) (width 0.28) (layer F.Cu) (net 40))
 (segment (start 134.62 132.43) (end 134.62 132.08) (width 0.28) (layer F.Cu) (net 40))
 (segment (start 146.05 132.08) (end 139.7 132.08) (width 0.28) (layer F.Cu) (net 39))
 (segment (start 104.14 132.08) (end 109.03 132.08) (width 0.28) (layer F.Cu) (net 42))
 (segment (start 109.03 132.08) (end 110.49 133.54) (width 0.28) (layer F.Cu) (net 42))
 (segment (start 110.49 133.54) (end 110.49 134.62) (width 0.28) (layer F.Cu) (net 42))
 (segment (start 129.54 144.78) (end 134.62 139.7) (width 0.28) (layer F.Cu) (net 37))
 (segment (start 129.54 144.78) (end 119.57 144.78) (width 0.28) (layer F.Cu) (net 37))
 (segment (start 119.57 144.78) (end 118.11 143.32) (width 0.28) (layer F.Cu) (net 37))
 (segment (start 118.11 143.32) (end 118.11 142.24) (width 0.28) (layer F.Cu) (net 37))
 (segment (start 119.6 138.56) (end 118.46 139.7) (width 0.28) (layer B.Cu) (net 38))
 (segment (start 118.46 139.7) (end 118.11 139.7) (width 0.28) (layer B.Cu) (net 38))
 (segment (start 104.14 135.89) (end 102.801 137.229) (width 0.28) (layer F.Cu) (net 38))
 (segment (start 102.801 137.229) (end 102.801 144.153) (width 0.28) (layer F.Cu) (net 38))
 (segment (start 102.801 144.153) (end 103.497 144.849) (width 0.28) (layer F.Cu) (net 38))
 (segment (start 103.497 144.849) (end 112.611 144.849) (width 0.28) (layer F.Cu) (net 38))
 (segment (start 112.611 144.849) (end 117.76 139.7) (width 0.28) (layer F.Cu) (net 38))
 (segment (start 117.76 139.7) (end 118.11 139.7) (width 0.28) (layer F.Cu) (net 38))
 (segment (start 119.6 138.56) (end 118.46 139.7) (width 0.28) (layer B.Cu) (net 38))
 (segment (start 139.7 139.7) (end 139.7 139.35) (width 0.28) (layer B.Cu) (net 38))
 (segment (start 139.7 139.35) (end 136.89 136.54) (width 0.28) (layer B.Cu) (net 38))
 (segment (start 136.89 136.54) (end 130.68 136.54) (width 0.28) (layer B.Cu) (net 38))
 (segment (start 130.68 136.54) (end 127.71 133.57) (width 0.28) (layer B.Cu) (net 38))
 (segment (start 127.71 133.57) (end 127.69 133.57) (width 0.28) (layer B.Cu) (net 38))
 (segment (start 127.69 133.57) (end 125.74 131.62) (width 0.28) (layer B.Cu) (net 38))
 (segment (start 125.74 131.62) (end 123.008 131.62) (width 0.28) (layer B.Cu) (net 38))
 (segment (start 123.008 131.62) (end 120.63 133.998) (width 0.28) (layer B.Cu) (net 38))
 (segment (start 120.63 133.998) (end 120.63 137.53) (width 0.28) (layer B.Cu) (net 38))
 (segment (start 120.63 137.53) (end 119.6 138.56) (width 0.28) (layer B.Cu) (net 38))
 (segment (start 104.14 139.7) (end 105.41 138.43) (width 0.28) (layer F.Cu) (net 7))
 (segment (start 105.41 138.43) (end 115.41 138.43) (width 0.28) (layer F.Cu) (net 7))
 (segment (start 115.41 138.43) (end 116.68 137.16) (width 0.28) (layer F.Cu) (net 7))
 (segment (start 116.68 137.16) (end 118.11 137.16) (width 0.28) (layer F.Cu) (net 7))
 (segment (start 104.14 143.51) (end 105.139 142.511) (width 0.28) (layer F.Cu) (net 7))
 (segment (start 105.139 142.511) (end 105.139 140.699) (width 0.28) (layer F.Cu) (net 7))
 (segment (start 105.139 140.699) (end 104.14 139.7) (width 0.28) (layer F.Cu) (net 7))
 (segment (start 118.11 137.16) (end 118.46 137.16) (width 0.28) (layer F.Cu) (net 7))
 (segment (start 101.39 127) (end 101.39 136.95) (width 0.28) (layer B.Cu) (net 7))
 (segment (start 101.39 136.95) (end 104.14 139.7) (width 0.28) (layer B.Cu) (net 7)))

